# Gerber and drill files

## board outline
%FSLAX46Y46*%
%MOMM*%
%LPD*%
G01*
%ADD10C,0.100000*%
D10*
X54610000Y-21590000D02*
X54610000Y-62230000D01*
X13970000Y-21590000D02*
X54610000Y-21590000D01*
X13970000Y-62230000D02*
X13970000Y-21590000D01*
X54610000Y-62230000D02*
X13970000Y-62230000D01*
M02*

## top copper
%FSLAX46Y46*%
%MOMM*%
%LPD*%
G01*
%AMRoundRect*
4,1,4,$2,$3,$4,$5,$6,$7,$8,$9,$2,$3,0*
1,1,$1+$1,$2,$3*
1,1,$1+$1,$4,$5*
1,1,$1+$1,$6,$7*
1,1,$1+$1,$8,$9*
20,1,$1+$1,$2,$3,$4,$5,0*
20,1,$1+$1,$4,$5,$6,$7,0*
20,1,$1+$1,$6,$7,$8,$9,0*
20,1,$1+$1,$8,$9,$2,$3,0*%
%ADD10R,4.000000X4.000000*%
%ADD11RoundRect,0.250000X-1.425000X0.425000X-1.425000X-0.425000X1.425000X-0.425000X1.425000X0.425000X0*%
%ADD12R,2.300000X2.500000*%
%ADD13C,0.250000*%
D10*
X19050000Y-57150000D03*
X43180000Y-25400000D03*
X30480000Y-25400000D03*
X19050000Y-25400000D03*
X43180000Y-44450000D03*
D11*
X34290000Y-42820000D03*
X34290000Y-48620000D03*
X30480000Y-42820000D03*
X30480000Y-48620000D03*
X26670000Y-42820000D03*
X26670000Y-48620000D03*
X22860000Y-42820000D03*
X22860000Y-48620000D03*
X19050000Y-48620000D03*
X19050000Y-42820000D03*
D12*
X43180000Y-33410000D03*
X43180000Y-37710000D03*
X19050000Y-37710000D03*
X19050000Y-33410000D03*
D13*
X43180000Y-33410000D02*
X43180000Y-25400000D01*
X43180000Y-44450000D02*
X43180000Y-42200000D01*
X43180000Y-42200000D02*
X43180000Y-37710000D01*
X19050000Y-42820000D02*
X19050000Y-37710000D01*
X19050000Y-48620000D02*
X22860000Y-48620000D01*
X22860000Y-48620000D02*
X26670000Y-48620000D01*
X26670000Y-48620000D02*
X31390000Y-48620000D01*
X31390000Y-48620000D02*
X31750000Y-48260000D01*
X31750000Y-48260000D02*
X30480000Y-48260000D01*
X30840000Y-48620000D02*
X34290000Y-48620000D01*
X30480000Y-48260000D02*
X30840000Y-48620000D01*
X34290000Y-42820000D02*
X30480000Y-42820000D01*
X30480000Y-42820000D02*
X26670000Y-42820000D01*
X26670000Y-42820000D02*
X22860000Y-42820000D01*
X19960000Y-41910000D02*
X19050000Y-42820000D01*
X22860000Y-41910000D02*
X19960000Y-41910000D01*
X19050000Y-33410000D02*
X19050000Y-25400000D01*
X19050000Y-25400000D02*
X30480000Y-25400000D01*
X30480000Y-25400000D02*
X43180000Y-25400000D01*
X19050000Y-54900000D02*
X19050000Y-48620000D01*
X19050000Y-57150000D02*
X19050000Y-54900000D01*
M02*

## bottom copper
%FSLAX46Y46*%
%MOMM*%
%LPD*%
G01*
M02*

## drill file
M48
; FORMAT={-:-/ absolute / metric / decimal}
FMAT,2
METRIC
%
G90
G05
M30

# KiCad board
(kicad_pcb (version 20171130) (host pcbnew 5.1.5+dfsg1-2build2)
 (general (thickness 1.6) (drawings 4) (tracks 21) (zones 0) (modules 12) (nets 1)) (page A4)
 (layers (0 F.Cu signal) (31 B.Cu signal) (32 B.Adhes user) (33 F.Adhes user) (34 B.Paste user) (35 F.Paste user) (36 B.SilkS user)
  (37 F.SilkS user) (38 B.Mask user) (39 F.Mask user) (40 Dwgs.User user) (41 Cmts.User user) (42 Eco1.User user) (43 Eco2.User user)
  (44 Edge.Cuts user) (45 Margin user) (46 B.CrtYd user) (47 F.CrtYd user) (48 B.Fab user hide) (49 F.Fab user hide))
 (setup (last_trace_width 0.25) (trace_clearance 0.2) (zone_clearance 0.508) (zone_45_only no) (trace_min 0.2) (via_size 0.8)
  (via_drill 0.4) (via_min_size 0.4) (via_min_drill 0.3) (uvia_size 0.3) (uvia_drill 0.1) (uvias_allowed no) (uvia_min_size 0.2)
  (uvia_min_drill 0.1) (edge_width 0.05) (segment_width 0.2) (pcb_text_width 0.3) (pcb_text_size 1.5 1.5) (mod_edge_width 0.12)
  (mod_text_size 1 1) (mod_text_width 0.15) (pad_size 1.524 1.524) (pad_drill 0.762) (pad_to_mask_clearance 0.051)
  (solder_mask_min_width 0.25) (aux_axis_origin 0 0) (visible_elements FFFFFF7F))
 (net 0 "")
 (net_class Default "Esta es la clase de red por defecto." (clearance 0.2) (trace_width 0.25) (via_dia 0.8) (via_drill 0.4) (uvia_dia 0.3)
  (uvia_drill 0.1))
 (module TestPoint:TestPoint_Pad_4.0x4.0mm (layer F.Cu) (at 19.05 57.15)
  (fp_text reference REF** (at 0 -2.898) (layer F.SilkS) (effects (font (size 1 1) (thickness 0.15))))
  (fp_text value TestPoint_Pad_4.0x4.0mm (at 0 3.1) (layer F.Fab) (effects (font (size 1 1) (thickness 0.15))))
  (pad 1 smd rect (at 0 0) (size 4 4) (layers F.Cu F.Mask)))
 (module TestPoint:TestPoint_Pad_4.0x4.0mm (layer F.Cu) (at 43.18 25.4)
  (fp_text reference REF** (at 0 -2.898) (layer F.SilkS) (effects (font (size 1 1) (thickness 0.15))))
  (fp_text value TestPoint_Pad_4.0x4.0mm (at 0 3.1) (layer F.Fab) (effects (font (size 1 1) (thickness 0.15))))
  (pad 1 smd rect (at 0 0) (size 4 4) (layers F.Cu F.Mask)))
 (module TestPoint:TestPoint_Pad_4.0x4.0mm (layer F.Cu) (at 30.48 25.4)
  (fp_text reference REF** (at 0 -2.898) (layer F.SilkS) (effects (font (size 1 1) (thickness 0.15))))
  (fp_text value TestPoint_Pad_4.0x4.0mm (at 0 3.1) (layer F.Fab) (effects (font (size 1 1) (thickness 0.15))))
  (pad 1 smd rect (at 0 0) (size 4 4) (layers F.Cu F.Mask)))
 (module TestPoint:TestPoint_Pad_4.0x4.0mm (layer F.Cu) (at 19.05 25.4)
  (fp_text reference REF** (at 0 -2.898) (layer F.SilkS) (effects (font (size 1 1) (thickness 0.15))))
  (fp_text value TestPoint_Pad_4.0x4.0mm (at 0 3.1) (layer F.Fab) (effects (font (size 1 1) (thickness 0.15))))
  (pad 1 smd rect (at 0 0) (size 4 4) (layers F.Cu F.Mask)))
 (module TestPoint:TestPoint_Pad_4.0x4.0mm (layer F.Cu) (at 43.18 44.45)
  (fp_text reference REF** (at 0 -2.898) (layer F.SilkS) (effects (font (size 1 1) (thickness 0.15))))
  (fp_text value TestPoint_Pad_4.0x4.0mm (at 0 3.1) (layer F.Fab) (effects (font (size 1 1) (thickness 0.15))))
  (pad 1 smd rect (at 0 0) (size 4 4) (layers F.Cu F.Mask)))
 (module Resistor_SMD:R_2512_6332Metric (layer F.Cu) (at 34.29 45.72 270)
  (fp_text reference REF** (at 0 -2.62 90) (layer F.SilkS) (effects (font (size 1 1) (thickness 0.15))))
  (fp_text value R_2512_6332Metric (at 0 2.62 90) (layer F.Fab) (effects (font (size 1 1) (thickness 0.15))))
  (pad 1 smd roundrect (at -2.9 0 270) (size 1.35 3.35) (layers F.Cu F.Paste F.Mask) (roundrect_rratio 0.185185))
  (pad 2 smd roundrect (at 2.9 0 270) (size 1.35 3.35) (layers F.Cu F.Paste F.Mask) (roundrect_rratio 0.185185)))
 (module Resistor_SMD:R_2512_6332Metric (layer F.Cu) (at 30.48 45.72 270)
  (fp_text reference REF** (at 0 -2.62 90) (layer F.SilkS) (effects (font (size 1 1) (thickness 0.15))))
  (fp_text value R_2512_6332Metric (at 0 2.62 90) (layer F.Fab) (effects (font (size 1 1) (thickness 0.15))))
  (pad 1 smd roundrect (at -2.9 0 270) (size 1.35 3.35) (layers F.Cu F.Paste F.Mask) (roundrect_rratio 0.185185))
  (pad 2 smd roundrect (at 2.9 0 270) (size 1.35 3.35) (layers F.Cu F.Paste F.Mask) (roundrect_rratio 0.185185)))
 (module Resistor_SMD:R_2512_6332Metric (layer F.Cu) (at 26.67 45.72 270)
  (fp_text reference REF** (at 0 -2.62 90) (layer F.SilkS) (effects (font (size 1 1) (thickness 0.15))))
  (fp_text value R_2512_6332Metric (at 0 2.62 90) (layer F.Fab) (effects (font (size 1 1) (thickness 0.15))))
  (pad 1 smd roundrect (at -2.9 0 270) (size 1.35 3.35) (layers F.Cu F.Paste F.Mask) (roundrect_rratio 0.185185))
  (pad 2 smd roundrect (at 2.9 0 270) (size 1.35 3.35) (layers F.Cu F.Paste F.Mask) (roundrect_rratio 0.185185)))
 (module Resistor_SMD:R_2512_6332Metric (layer F.Cu) (at 22.86 45.72 270)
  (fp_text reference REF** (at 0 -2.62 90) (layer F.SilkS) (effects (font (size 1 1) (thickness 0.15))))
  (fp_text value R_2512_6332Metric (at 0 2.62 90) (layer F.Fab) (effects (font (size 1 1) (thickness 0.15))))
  (pad 1 smd roundrect (at -2.9 0 270) (size 1.35 3.35) (layers F.Cu F.Paste F.Mask) (roundrect_rratio 0.185185))
  (pad 2 smd roundrect (at 2.9 0 270) (size 1.35 3.35) (layers F.Cu F.Paste F.Mask) (roundrect_rratio 0.185185)))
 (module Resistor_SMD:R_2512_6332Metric (layer F.Cu) (at 19.05 45.72 270)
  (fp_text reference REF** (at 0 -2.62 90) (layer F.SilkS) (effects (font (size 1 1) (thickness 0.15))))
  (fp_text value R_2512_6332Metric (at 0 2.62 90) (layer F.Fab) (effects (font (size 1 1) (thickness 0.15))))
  (pad 2 smd roundrect (at 2.9 0 270) (size 1.35 3.35) (layers F.Cu F.Paste F.Mask) (roundrect_rratio 0.185185))
  (pad 1 smd roundrect (at -2.9 0 270) (size 1.35 3.35) (layers F.Cu F.Paste F.Mask) (roundrect_rratio 0.185185)))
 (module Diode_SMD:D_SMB (layer F.Cu) (at 43.18 35.56 270)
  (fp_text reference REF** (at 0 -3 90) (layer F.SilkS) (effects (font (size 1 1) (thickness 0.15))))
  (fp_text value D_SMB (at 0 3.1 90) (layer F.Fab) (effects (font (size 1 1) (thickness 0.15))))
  (pad 1 smd rect (at -2.15 0 270) (size 2.5 2.3) (layers F.Cu F.Paste F.Mask))
  (pad 2 smd rect (at 2.15 0 270) (size 2.5 2.3) (layers F.Cu F.Paste F.Mask)))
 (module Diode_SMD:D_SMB (layer F.Cu) (at 19.05 35.56 270)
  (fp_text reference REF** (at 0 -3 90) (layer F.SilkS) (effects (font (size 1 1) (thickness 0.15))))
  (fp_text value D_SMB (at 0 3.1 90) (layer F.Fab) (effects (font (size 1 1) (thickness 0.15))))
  (pad 2 smd rect (at 2.15 0 270) (size 2.5 2.3) (layers F.Cu F.Paste F.Mask))
  (pad 1 smd rect (at -2.15 0 270) (size 2.5 2.3) (layers F.Cu F.Paste F.Mask)))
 (gr_line (start 54.61 21.59) (end 54.61 62.23) (layer Edge.Cuts) (width 0.1))
 (gr_line (start 13.97 21.59) (end 54.61 21.59) (layer Edge.Cuts) (width 0.1))
 (gr_line (start 13.97 62.23) (end 13.97 21.59) (layer Edge.Cuts) (width 0.1))
 (gr_line (start 54.61 62.23) (end 13.97 62.23) (layer Edge.Cuts) (width 0.1))
 (segment (start 43.18 33.41) (end 43.18 25.4) (width 0.25) (layer F.Cu) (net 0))
 (segment (start 43.18 44.45) (end 43.18 42.2) (width 0.25) (layer F.Cu) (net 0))
 (segment (start 43.18 42.2) (end 43.18 37.71) (width 0.25) (layer F.Cu) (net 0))
 (segment (start 19.05 42.82) (end 19.05 37.71) (width 0.25) (layer F.Cu) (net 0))
 (segment (start 19.05 48.62) (end 22.86 48.62) (width 0.25) (layer F.Cu) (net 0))
 (segment (start 22.86 48.62) (end 26.67 48.62) (width 0.25) (layer F.Cu) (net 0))
 (segment (start 26.67 48.62) (end 31.39 48.62) (width 0.25) (layer F.Cu) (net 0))
 (segment (start 31.39 48.62) (end 31.75 48.26) (width 0.25) (layer F.Cu) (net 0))
 (segment (start 31.75 48.26) (end 30.48 48.26) (width 0.25) (layer F.Cu) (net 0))
 (segment (start 30.84 48.62) (end 34.29 48.62) (width 0.25) (layer F.Cu) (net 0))
 (segment (start 30.48 48.26) (end 30.84 48.62) (width 0.25) (layer F.Cu) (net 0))
 (segment (start 34.29 42.82) (end 30.48 42.82) (width 0.25) (layer F.Cu) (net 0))
 (segment (start 30.48 42.82) (end 26.67 42.82) (width 0.25) (layer F.Cu) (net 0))
 (segment (start 26.67 42.82) (end 22.86 42.82) (width 0.25) (layer F.Cu) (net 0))
 (segment (start 19.96 41.91) (end 19.05 42.82) (width 0.25) (layer F.Cu) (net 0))
 (segment (start 22.86 41.91) (end 19.96 41.91) (width 0.25) (layer F.Cu) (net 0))
 (segment (start 19.05 33.41) (end 19.05 25.4) (width 0.25) (layer F.Cu) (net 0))
 (segment (start 19.05 25.4) (end 30.48 25.4) (width 0.25) (layer F.Cu) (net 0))
 (segment (start 30.48 25.4) (end 43.18 25.4) (width 0.25) (layer F.Cu) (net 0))
 (segment (start 19.05 54.9) (end 19.05 48.62) (width 0.25) (layer F.Cu) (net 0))
 (segment (start 19.05 57.15) (end 19.05 54.9) (width 0.25) (layer F.Cu) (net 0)))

